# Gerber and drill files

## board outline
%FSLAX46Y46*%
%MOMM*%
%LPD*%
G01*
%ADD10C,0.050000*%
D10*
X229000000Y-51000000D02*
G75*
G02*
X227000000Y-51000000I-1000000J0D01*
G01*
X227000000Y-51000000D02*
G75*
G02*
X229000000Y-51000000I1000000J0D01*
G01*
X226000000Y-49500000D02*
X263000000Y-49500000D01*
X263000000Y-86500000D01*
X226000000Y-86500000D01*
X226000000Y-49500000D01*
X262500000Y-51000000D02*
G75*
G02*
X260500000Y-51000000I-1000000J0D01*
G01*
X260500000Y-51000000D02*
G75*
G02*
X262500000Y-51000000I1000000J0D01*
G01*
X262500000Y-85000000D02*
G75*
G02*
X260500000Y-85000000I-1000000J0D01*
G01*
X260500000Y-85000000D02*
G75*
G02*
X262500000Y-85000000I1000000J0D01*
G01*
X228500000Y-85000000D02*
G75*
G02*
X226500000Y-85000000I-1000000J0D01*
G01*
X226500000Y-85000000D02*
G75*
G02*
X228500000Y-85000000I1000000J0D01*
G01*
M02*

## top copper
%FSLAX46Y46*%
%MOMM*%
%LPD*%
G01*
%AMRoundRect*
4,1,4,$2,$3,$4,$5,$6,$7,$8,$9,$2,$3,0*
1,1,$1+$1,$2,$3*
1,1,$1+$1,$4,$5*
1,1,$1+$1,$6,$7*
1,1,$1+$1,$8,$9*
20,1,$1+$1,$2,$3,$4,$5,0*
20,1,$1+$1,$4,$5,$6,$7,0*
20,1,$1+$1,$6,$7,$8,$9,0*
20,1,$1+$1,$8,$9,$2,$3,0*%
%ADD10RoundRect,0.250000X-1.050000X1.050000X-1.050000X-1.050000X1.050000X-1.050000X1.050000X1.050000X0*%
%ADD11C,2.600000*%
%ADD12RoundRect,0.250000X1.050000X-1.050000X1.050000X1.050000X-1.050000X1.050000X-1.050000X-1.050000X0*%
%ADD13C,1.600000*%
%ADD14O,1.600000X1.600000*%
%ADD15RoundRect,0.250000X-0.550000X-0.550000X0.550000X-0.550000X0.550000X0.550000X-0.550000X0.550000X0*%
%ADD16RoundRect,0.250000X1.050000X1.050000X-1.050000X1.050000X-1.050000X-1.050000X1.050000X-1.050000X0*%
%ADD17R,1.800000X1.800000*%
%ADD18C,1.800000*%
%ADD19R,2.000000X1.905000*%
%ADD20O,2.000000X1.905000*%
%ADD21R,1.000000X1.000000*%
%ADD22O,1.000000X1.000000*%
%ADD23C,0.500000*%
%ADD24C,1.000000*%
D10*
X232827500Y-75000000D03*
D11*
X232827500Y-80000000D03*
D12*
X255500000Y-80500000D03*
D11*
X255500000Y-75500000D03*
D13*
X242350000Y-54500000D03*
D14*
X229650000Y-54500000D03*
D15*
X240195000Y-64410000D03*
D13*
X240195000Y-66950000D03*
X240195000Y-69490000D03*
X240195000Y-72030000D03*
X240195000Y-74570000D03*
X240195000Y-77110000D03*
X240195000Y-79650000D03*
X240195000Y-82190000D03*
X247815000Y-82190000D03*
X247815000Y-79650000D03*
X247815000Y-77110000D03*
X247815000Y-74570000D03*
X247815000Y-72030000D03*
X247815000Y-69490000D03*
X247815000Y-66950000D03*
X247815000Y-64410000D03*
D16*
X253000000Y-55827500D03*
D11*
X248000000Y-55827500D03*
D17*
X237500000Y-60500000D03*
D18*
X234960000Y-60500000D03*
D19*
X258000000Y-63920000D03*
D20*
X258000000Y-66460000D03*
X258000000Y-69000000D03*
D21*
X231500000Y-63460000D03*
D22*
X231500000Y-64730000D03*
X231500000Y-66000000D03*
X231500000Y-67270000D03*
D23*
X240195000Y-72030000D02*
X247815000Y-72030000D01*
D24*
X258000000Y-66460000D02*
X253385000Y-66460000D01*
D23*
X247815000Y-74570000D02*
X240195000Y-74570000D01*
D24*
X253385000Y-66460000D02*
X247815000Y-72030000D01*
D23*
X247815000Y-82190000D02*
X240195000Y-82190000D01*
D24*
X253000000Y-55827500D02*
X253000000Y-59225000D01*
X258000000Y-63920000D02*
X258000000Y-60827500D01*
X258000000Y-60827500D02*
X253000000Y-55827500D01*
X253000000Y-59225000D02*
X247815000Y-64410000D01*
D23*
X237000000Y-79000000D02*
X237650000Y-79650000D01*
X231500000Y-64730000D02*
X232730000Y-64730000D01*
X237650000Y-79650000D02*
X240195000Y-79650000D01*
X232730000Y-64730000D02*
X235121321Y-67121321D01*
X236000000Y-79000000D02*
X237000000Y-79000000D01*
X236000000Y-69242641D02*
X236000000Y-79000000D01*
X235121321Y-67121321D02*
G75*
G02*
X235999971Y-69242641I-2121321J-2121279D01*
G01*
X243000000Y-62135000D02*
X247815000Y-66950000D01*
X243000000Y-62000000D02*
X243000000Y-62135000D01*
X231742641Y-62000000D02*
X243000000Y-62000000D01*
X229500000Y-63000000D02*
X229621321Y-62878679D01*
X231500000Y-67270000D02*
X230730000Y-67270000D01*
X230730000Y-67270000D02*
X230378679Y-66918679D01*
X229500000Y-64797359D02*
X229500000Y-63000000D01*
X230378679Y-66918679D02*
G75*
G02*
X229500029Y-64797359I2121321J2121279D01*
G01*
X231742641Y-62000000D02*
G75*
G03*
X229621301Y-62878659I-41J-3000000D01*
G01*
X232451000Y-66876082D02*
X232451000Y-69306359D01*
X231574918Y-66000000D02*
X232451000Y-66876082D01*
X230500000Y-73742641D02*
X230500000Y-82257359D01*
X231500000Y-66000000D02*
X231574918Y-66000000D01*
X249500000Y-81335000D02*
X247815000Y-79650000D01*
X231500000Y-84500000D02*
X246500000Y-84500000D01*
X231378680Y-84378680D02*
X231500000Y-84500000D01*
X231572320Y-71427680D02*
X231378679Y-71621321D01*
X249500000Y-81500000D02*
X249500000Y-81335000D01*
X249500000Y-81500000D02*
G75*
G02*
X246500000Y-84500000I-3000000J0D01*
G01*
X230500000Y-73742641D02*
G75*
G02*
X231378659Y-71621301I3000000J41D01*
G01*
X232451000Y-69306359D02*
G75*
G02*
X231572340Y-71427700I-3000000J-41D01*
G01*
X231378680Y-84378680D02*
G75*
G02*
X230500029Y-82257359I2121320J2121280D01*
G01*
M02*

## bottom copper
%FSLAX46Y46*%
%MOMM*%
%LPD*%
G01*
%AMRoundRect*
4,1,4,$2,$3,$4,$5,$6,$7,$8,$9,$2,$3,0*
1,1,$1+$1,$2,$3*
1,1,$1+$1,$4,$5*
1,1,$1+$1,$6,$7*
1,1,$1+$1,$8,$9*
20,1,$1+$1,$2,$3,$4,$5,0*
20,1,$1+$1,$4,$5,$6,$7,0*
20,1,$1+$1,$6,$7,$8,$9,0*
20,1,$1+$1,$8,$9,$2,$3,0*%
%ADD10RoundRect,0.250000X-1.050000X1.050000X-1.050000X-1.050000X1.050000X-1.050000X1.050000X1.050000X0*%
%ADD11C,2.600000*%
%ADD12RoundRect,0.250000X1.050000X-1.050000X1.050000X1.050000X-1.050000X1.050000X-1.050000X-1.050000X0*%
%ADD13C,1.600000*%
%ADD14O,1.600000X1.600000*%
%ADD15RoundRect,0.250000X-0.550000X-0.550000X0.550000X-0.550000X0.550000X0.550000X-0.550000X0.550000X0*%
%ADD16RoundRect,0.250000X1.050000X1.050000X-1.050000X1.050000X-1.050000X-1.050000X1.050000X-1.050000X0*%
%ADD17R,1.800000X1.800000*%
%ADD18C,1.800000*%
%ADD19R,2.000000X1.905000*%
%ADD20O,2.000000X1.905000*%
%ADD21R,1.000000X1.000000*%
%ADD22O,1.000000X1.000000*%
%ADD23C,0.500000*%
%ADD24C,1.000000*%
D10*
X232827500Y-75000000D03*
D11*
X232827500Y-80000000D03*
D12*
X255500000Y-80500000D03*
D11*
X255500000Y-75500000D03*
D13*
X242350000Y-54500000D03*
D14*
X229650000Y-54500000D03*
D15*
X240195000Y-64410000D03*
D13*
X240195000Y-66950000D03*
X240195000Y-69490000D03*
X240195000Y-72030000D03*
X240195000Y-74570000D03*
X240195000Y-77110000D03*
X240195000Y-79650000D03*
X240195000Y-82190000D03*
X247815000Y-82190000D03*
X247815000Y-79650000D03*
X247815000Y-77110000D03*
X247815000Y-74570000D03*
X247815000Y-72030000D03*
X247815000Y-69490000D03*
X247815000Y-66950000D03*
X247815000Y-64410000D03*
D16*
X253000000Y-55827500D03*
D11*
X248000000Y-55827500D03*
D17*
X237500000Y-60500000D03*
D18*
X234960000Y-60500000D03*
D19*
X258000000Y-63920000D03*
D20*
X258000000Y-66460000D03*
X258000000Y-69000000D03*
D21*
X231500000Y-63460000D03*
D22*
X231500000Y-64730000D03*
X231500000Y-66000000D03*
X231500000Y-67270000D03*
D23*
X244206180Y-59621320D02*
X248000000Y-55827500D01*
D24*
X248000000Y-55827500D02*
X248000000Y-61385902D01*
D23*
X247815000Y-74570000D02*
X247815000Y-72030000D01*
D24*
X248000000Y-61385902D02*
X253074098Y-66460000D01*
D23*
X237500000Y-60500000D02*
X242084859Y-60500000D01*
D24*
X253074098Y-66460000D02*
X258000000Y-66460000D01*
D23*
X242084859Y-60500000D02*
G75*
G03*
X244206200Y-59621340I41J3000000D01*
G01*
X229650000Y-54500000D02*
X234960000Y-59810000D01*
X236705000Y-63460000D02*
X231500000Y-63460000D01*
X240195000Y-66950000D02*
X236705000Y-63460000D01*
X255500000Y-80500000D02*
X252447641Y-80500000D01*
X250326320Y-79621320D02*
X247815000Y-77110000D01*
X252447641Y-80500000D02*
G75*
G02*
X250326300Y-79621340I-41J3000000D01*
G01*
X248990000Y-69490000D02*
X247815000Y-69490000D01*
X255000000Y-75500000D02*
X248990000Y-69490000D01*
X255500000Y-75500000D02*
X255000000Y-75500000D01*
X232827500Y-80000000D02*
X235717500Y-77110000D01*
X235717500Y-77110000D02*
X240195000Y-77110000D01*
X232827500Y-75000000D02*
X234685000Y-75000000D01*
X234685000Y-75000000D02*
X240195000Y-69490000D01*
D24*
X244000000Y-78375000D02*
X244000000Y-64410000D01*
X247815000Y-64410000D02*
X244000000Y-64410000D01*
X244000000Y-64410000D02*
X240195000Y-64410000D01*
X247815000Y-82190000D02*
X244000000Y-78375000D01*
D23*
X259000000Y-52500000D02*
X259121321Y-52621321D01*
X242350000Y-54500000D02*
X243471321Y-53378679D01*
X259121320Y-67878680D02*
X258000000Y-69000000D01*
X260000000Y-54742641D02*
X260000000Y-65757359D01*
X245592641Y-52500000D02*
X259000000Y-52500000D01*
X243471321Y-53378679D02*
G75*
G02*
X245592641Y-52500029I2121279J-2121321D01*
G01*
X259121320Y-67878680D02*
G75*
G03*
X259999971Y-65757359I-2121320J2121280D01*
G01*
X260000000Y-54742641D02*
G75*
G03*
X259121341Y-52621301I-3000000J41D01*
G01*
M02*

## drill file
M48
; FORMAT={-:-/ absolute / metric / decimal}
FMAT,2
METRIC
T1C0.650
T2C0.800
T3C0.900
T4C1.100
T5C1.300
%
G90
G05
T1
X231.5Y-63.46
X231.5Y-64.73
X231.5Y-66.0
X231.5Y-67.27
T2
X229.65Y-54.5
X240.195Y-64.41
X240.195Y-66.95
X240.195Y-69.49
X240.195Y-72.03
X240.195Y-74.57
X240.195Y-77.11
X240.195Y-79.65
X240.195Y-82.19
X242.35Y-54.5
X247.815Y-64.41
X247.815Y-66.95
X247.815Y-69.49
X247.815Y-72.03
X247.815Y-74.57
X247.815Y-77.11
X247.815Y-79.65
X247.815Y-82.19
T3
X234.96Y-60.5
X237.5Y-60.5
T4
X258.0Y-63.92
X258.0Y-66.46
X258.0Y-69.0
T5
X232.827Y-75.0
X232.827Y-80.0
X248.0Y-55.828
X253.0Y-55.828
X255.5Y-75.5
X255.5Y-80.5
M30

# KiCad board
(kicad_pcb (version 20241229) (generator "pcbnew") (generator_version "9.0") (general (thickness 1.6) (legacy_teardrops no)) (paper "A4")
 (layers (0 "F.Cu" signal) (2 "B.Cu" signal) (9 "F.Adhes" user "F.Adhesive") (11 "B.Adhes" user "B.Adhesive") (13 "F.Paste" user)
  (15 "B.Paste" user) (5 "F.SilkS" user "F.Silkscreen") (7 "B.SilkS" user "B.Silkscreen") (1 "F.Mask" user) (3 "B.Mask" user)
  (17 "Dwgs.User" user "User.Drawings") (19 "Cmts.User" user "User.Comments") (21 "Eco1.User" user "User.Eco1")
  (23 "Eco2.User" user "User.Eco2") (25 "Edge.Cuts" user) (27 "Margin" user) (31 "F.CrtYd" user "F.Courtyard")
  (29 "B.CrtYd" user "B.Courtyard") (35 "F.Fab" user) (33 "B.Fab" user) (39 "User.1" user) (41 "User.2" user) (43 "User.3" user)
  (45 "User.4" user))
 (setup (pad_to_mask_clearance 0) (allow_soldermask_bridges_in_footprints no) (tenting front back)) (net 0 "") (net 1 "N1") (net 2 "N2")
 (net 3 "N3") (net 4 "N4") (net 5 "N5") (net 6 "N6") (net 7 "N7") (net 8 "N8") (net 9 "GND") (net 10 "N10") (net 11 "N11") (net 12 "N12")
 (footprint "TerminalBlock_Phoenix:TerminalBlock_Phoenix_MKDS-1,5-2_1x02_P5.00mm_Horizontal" (layer "F.Cu") (at 232.8275 75 -90)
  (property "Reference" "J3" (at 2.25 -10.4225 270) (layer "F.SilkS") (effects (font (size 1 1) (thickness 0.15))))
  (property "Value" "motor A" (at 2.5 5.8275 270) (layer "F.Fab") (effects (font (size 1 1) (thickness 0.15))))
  (pad "1" thru_hole roundrect (at 0 0 270) (size 2.6 2.6) (drill 1.3) (layers "*.Cu" "*.Mask") (remove_unused_layers no)
   (roundrect_rratio 0.096154) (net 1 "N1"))
  (pad "2" thru_hole circle (at 5 0 270) (size 2.6 2.6) (drill 1.3) (layers "*.Cu" "*.Mask") (remove_unused_layers no) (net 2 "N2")))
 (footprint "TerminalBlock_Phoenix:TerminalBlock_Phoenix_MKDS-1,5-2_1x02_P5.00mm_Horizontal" (layer "F.Cu") (at 255.5 80.5 90)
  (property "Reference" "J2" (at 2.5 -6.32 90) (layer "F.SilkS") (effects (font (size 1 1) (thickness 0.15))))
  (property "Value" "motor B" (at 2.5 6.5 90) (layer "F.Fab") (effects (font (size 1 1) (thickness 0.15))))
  (pad "1" thru_hole roundrect (at 0 0 90) (size 2.6 2.6) (drill 1.3) (layers "*.Cu" "*.Mask") (remove_unused_layers no)
   (roundrect_rratio 0.096154) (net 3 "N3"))
  (pad "2" thru_hole circle (at 5 0 90) (size 2.6 2.6) (drill 1.3) (layers "*.Cu" "*.Mask") (remove_unused_layers no) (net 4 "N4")))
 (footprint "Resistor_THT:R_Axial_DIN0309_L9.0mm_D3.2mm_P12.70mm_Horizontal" (layer "F.Cu") (at 242.35 54.5 180)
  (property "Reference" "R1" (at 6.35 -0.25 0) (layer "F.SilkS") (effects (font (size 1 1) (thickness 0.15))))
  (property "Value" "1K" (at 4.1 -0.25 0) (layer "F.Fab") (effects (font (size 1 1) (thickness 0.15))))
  (pad "1" thru_hole circle (at 0 0 180) (size 1.6 1.6) (drill 0.8) (layers "*.Cu" "*.Mask") (remove_unused_layers no) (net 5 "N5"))
  (pad "2" thru_hole oval (at 12.7 0 180) (size 1.6 1.6) (drill 0.8) (layers "*.Cu" "*.Mask") (remove_unused_layers no) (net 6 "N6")))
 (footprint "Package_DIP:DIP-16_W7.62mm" (layer "F.Cu") (at 240.195 64.41)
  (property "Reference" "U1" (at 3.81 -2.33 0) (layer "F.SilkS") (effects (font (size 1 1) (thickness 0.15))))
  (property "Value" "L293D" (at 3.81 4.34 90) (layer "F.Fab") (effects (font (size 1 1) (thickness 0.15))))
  (pad "1" thru_hole roundrect (at 0 0) (size 1.6 1.6) (drill 0.8) (layers "*.Cu" "*.Mask") (remove_unused_layers no)
   (roundrect_rratio 0.15625) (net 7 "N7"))
  (pad "2" thru_hole circle (at 0 2.54) (size 1.6 1.6) (drill 0.8) (layers "*.Cu" "*.Mask") (remove_unused_layers no) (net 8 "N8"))
  (pad "3" thru_hole circle (at 0 5.08) (size 1.6 1.6) (drill 0.8) (layers "*.Cu" "*.Mask") (remove_unused_layers no) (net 1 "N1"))
  (pad "4" thru_hole circle (at 0 7.62) (size 1.6 1.6) (drill 0.8) (layers "*.Cu" "*.Mask") (remove_unused_layers no) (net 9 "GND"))
  (pad "5" thru_hole circle (at 0 10.16) (size 1.6 1.6) (drill 0.8) (layers "*.Cu" "*.Mask") (remove_unused_layers no) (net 9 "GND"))
  (pad "6" thru_hole circle (at 0 12.7) (size 1.6 1.6) (drill 0.8) (layers "*.Cu" "*.Mask") (remove_unused_layers no) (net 2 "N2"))
  (pad "7" thru_hole circle (at 0 15.24) (size 1.6 1.6) (drill 0.8) (layers "*.Cu" "*.Mask") (remove_unused_layers no) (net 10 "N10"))
  (pad "8" thru_hole circle (at 0 17.78) (size 1.6 1.6) (drill 0.8) (layers "*.Cu" "*.Mask") (remove_unused_layers no) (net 7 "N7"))
  (pad "9" thru_hole circle (at 7.62 17.78) (size 1.6 1.6) (drill 0.8) (layers "*.Cu" "*.Mask") (remove_unused_layers no) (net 7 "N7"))
  (pad "10" thru_hole circle (at 7.62 15.24) (size 1.6 1.6) (drill 0.8) (layers "*.Cu" "*.Mask") (remove_unused_layers no) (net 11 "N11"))
  (pad "11" thru_hole circle (at 7.62 12.7) (size 1.6 1.6) (drill 0.8) (layers "*.Cu" "*.Mask") (remove_unused_layers no) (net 3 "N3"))
  (pad "12" thru_hole circle (at 7.62 10.16) (size 1.6 1.6) (drill 0.8) (layers "*.Cu" "*.Mask") (remove_unused_layers no) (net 9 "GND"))
  (pad "13" thru_hole circle (at 7.62 7.62) (size 1.6 1.6) (drill 0.8) (layers "*.Cu" "*.Mask") (remove_unused_layers no) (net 9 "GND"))
  (pad "14" thru_hole circle (at 7.62 5.08) (size 1.6 1.6) (drill 0.8) (layers "*.Cu" "*.Mask") (remove_unused_layers no) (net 4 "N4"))
  (pad "15" thru_hole circle (at 7.62 2.54) (size 1.6 1.6) (drill 0.8) (layers "*.Cu" "*.Mask") (remove_unused_layers no) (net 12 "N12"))
  (pad "16" thru_hole circle (at 7.62 0) (size 1.6 1.6) (drill 0.8) (layers "*.Cu" "*.Mask") (remove_unused_layers no) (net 7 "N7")))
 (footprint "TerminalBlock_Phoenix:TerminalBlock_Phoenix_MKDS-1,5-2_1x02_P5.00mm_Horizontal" (layer "F.Cu") (at 253 55.8275 180)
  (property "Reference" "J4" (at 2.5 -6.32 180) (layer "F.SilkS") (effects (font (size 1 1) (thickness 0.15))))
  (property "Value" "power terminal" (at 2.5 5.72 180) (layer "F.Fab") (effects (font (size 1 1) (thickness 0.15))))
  (pad "1" thru_hole roundrect (at 0 0 180) (size 2.6 2.6) (drill 1.3) (layers "*.Cu" "*.Mask") (remove_unused_layers no)
   (roundrect_rratio 0.096154) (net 7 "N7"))
  (pad "2" thru_hole circle (at 5 0 180) (size 2.6 2.6) (drill 1.3) (layers "*.Cu" "*.Mask") (remove_unused_layers no) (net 9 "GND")))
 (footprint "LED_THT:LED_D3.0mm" (layer "F.Cu") (at 237.5 60.5 180)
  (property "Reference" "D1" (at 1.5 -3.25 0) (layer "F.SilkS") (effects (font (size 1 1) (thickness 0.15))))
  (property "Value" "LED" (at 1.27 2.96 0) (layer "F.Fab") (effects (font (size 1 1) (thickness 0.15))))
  (pad "1" thru_hole rect (at 0 0 180) (size 1.8 1.8) (drill 0.9) (layers "*.Cu" "*.Mask") (remove_unused_layers no) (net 9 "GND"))
  (pad "2" thru_hole circle (at 2.54 0 180) (size 1.8 1.8) (drill 0.9) (layers "*.Cu" "*.Mask") (remove_unused_layers no) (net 6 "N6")))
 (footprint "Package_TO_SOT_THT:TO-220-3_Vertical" (layer "F.Cu") (at 258 63.92 -90)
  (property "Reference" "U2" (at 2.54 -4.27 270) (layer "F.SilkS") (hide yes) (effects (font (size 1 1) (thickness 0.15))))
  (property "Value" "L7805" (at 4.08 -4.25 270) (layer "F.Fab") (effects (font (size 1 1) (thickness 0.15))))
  (pad "1" thru_hole rect (at 0 0 270) (size 1.905 2) (drill 1.1) (layers "*.Cu" "*.Mask") (remove_unused_layers no) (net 7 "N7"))
  (pad "2" thru_hole oval (at 2.54 0 270) (size 1.905 2) (drill 1.1) (layers "*.Cu" "*.Mask") (remove_unused_layers no) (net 9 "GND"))
  (pad "3" thru_hole oval (at 5.08 0 270) (size 1.905 2) (drill 1.1) (layers "*.Cu" "*.Mask") (remove_unused_layers no) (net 5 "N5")))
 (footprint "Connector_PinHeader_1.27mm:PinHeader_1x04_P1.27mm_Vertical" (layer "F.Cu") (at 231.5 63.46)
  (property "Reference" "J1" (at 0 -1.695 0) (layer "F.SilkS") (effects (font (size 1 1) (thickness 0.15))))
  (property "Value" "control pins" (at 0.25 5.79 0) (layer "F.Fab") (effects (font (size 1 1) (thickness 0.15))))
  (pad "1" thru_hole rect (at 0 0) (size 1 1) (drill 0.65) (layers "*.Cu" "*.Mask") (remove_unused_layers no) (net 8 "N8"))
  (pad "2" thru_hole oval (at 0 1.27) (size 1 1) (drill 0.65) (layers "*.Cu" "*.Mask") (remove_unused_layers no) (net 10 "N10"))
  (pad "3" thru_hole oval (at 0 2.54) (size 1 1) (drill 0.65) (layers "*.Cu" "*.Mask") (remove_unused_layers no) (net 11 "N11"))
  (pad "4" thru_hole oval (at 0 3.81) (size 1 1) (drill 0.65) (layers "*.Cu" "*.Mask") (remove_unused_layers no) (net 12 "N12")))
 (gr_circle (center 228 51) (end 229 51) (stroke (width 0.05) (type default)) (fill no) (layer "Edge.Cuts"))
 (gr_rect (start 226 49.5) (end 263 86.5) (stroke (width 0.05) (type solid)) (fill no) (locked yes) (layer "Edge.Cuts"))
 (gr_circle (center 261.5 51) (end 262.5 51) (stroke (width 0.05) (type default)) (fill no) (layer "Edge.Cuts"))
 (gr_circle (center 261.5 85) (end 262.5 85) (stroke (width 0.05) (type default)) (fill no) (layer "Edge.Cuts"))
 (gr_circle (center 227.5 85) (end 228.5 85) (stroke (width 0.05) (type default)) (fill no) (layer "Edge.Cuts"))
 (segment (start 240.195 72.03) (end 247.815 72.03) (width 0.5) (layer "F.Cu") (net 9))
 (segment (start 258 66.46) (end 253.385 66.46) (width 1) (layer "F.Cu") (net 9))
 (segment (start 247.815 74.57) (end 240.195 74.57) (width 0.5) (layer "F.Cu") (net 9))
 (segment (start 253.385 66.46) (end 247.815 72.03) (width 1) (layer "F.Cu") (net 9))
 (segment (start 244.20618 59.62132) (end 248 55.8275) (width 0.5) (layer "B.Cu") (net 9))
 (segment (start 248 55.8275) (end 248 61.385902) (width 1) (layer "B.Cu") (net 9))
 (segment (start 247.815 74.57) (end 247.815 72.03) (width 0.5) (layer "B.Cu") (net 9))
 (segment (start 248 61.385902) (end 253.074098 66.46) (width 1) (layer "B.Cu") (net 9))
 (segment (start 237.5 60.5) (end 242.084859 60.5) (width 0.5) (layer "B.Cu") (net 9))
 (segment (start 253.074098 66.46) (end 258 66.46) (width 1) (layer "B.Cu") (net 9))
 (arc (start 242.084859 60.5) (mid 243.23291 60.271638) (end 244.20618 59.62132) (width 0.5) (layer "B.Cu") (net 9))
 (segment (start 229.65 54.5) (end 234.96 59.81) (width 0.5) (layer "B.Cu") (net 6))
 (segment (start 236.705 63.46) (end 231.5 63.46) (width 0.5) (layer "B.Cu") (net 8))
 (segment (start 240.195 66.95) (end 236.705 63.46) (width 0.5) (layer "B.Cu") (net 8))
 (segment (start 255.5 80.5) (end 252.447641 80.5) (width 0.5) (layer "B.Cu") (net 3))
 (segment (start 250.32632 79.62132) (end 247.815 77.11) (width 0.5) (layer "B.Cu") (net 3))
 (arc (start 252.447641 80.5) (mid 251.29959 80.271638) (end 250.32632 79.62132) (width 0.5) (layer "B.Cu") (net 3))
 (segment (start 248.99 69.49) (end 247.815 69.49) (width 0.5) (layer "B.Cu") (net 4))
 (segment (start 255 75.5) (end 248.99 69.49) (width 0.5) (layer "B.Cu") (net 4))
 (segment (start 255.5 75.5) (end 255 75.5) (width 0.5) (layer "B.Cu") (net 4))
 (segment (start 232.8275 80) (end 235.7175 77.11) (width 0.5) (layer "B.Cu") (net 2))
 (segment (start 235.7175 77.11) (end 240.195 77.11) (width 0.5) (layer "B.Cu") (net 2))
 (segment (start 232.8275 75) (end 234.685 75) (width 0.5) (layer "B.Cu") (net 1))
 (segment (start 234.685 75) (end 240.195 69.49) (width 0.5) (layer "B.Cu") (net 1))
 (segment (start 247.815 82.19) (end 240.195 82.19) (width 0.5) (layer "F.Cu") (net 7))
 (segment (start 253 55.8275) (end 253 59.225) (width 1) (layer "F.Cu") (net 7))
 (segment (start 258 63.92) (end 258 60.8275) (width 1) (layer "F.Cu") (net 7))
 (segment (start 258 60.8275) (end 253 55.8275) (width 1) (layer "F.Cu") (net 7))
 (segment (start 253 59.225) (end 247.815 64.41) (width 1) (layer "F.Cu") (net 7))
 (segment (start 244 78.375) (end 244 64.41) (width 1) (layer "B.Cu") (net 7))
 (segment (start 247.815 64.41) (end 244 64.41) (width 1) (layer "B.Cu") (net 7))
 (segment (start 244 64.41) (end 240.195 64.41) (width 1) (layer "B.Cu") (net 7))
 (segment (start 247.815 82.19) (end 244 78.375) (width 1) (layer "B.Cu") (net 7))
 (segment (start 259 52.5) (end 259.121321 52.621321) (width 0.5) (layer "B.Cu") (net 5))
 (segment (start 242.35 54.5) (end 243.471321 53.378679) (width 0.5) (layer "B.Cu") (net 5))
 (segment (start 259.12132 67.87868) (end 258 69) (width 0.5) (layer "B.Cu") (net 5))
 (segment (start 260 54.742641) (end 260 65.757359) (width 0.5) (layer "B.Cu") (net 5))
 (segment (start 245.592641 52.5) (end 259 52.5) (width 0.5) (layer "B.Cu") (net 5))
 (arc (start 243.471321 53.378679) (mid 244.444591 52.728361) (end 245.592641 52.5) (width 0.5) (layer "B.Cu") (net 5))
 (arc (start 259.12132 67.87868) (mid 259.771639 66.90541) (end 260 65.757359) (width 0.5) (layer "B.Cu") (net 5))
 (arc (start 260 54.742641) (mid 259.771639 53.594591) (end 259.121321 52.621321) (width 0.5) (layer "B.Cu") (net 5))
 (segment (start 237 79) (end 237.65 79.65) (width 0.5) (layer "F.Cu") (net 10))
 (segment (start 231.5 64.73) (end 232.73 64.73) (width 0.5) (layer "F.Cu") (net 10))
 (segment (start 237.65 79.65) (end 240.195 79.65) (width 0.5) (layer "F.Cu") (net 10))
 (segment (start 232.73 64.73) (end 235.121321 67.121321) (width 0.5) (layer "F.Cu") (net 10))
 (segment (start 236 79) (end 237 79) (width 0.5) (layer "F.Cu") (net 10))
 (segment (start 236 69.242641) (end 236 79) (width 0.5) (layer "F.Cu") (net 10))
 (arc (start 235.121321 67.121321) (mid 235.771639 68.094591) (end 236 69.242641) (width 0.5) (layer "F.Cu") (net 10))
 (segment (start 243 62.135) (end 247.815 66.95) (width 0.5) (layer "F.Cu") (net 12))
 (segment (start 243 62) (end 243 62.135) (width 0.5) (layer "F.Cu") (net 12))
 (segment (start 231.742641 62) (end 243 62) (width 0.5) (layer "F.Cu") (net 12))
 (segment (start 229.5 63) (end 229.621321 62.878679) (width 0.5) (layer "F.Cu") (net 12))
 (segment (start 231.5 67.27) (end 230.73 67.27) (width 0.5) (layer "F.Cu") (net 12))
 (segment (start 230.73 67.27) (end 230.378679 66.918679) (width 0.5) (layer "F.Cu") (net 12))
 (segment (start 229.5 64.797359) (end 229.5 63) (width 0.5) (layer "F.Cu") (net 12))
 (arc (start 230.378679 66.918679) (mid 229.728361 65.945409) (end 229.5 64.797359) (width 0.5) (layer "F.Cu") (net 12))
 (arc (start 231.742641 62) (mid 230.594591 62.228361) (end 229.621321 62.878679) (width 0.5) (layer "F.Cu") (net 12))
 (segment (start 232.451 66.876082) (end 232.451 69.306359) (width 0.5) (layer "F.Cu") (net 11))
 (segment (start 231.574918 66) (end 232.451 66.876082) (width 0.5) (layer "F.Cu") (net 11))
 (segment (start 230.5 73.742641) (end 230.5 82.257359) (width 0.5) (layer "F.Cu") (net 11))
 (segment (start 231.5 66) (end 231.574918 66) (width 0.5) (layer "F.Cu") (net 11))
 (segment (start 249.5 81.335) (end 247.815 79.65) (width 0.5) (layer "F.Cu") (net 11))
 (segment (start 231.5 84.5) (end 246.5 84.5) (width 0.5) (layer "F.Cu") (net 11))
 (segment (start 231.37868 84.37868) (end 231.5 84.5) (width 0.5) (layer "F.Cu") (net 11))
 (segment (start 231.57232 71.42768) (end 231.378679 71.621321) (width 0.5) (layer "F.Cu") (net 11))
 (segment (start 249.5 81.5) (end 249.5 81.335) (width 0.5) (layer "F.Cu") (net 11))
 (arc (start 249.5 81.5) (mid 248.62132 83.62132) (end 246.5 84.5) (width 0.5) (layer "F.Cu") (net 11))
 (arc (start 230.5 73.742641) (mid 230.728361 72.594591) (end 231.378679 71.621321) (width 0.5) (layer "F.Cu") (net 11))
 (arc (start 232.451 69.306359) (mid 232.222638 70.45441) (end 231.57232 71.42768) (width 0.5) (layer "F.Cu") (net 11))
 (arc (start 231.37868 84.37868) (mid 230.728361 83.40541) (end 230.5 82.257359) (width 0.5) (layer "F.Cu") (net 11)))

